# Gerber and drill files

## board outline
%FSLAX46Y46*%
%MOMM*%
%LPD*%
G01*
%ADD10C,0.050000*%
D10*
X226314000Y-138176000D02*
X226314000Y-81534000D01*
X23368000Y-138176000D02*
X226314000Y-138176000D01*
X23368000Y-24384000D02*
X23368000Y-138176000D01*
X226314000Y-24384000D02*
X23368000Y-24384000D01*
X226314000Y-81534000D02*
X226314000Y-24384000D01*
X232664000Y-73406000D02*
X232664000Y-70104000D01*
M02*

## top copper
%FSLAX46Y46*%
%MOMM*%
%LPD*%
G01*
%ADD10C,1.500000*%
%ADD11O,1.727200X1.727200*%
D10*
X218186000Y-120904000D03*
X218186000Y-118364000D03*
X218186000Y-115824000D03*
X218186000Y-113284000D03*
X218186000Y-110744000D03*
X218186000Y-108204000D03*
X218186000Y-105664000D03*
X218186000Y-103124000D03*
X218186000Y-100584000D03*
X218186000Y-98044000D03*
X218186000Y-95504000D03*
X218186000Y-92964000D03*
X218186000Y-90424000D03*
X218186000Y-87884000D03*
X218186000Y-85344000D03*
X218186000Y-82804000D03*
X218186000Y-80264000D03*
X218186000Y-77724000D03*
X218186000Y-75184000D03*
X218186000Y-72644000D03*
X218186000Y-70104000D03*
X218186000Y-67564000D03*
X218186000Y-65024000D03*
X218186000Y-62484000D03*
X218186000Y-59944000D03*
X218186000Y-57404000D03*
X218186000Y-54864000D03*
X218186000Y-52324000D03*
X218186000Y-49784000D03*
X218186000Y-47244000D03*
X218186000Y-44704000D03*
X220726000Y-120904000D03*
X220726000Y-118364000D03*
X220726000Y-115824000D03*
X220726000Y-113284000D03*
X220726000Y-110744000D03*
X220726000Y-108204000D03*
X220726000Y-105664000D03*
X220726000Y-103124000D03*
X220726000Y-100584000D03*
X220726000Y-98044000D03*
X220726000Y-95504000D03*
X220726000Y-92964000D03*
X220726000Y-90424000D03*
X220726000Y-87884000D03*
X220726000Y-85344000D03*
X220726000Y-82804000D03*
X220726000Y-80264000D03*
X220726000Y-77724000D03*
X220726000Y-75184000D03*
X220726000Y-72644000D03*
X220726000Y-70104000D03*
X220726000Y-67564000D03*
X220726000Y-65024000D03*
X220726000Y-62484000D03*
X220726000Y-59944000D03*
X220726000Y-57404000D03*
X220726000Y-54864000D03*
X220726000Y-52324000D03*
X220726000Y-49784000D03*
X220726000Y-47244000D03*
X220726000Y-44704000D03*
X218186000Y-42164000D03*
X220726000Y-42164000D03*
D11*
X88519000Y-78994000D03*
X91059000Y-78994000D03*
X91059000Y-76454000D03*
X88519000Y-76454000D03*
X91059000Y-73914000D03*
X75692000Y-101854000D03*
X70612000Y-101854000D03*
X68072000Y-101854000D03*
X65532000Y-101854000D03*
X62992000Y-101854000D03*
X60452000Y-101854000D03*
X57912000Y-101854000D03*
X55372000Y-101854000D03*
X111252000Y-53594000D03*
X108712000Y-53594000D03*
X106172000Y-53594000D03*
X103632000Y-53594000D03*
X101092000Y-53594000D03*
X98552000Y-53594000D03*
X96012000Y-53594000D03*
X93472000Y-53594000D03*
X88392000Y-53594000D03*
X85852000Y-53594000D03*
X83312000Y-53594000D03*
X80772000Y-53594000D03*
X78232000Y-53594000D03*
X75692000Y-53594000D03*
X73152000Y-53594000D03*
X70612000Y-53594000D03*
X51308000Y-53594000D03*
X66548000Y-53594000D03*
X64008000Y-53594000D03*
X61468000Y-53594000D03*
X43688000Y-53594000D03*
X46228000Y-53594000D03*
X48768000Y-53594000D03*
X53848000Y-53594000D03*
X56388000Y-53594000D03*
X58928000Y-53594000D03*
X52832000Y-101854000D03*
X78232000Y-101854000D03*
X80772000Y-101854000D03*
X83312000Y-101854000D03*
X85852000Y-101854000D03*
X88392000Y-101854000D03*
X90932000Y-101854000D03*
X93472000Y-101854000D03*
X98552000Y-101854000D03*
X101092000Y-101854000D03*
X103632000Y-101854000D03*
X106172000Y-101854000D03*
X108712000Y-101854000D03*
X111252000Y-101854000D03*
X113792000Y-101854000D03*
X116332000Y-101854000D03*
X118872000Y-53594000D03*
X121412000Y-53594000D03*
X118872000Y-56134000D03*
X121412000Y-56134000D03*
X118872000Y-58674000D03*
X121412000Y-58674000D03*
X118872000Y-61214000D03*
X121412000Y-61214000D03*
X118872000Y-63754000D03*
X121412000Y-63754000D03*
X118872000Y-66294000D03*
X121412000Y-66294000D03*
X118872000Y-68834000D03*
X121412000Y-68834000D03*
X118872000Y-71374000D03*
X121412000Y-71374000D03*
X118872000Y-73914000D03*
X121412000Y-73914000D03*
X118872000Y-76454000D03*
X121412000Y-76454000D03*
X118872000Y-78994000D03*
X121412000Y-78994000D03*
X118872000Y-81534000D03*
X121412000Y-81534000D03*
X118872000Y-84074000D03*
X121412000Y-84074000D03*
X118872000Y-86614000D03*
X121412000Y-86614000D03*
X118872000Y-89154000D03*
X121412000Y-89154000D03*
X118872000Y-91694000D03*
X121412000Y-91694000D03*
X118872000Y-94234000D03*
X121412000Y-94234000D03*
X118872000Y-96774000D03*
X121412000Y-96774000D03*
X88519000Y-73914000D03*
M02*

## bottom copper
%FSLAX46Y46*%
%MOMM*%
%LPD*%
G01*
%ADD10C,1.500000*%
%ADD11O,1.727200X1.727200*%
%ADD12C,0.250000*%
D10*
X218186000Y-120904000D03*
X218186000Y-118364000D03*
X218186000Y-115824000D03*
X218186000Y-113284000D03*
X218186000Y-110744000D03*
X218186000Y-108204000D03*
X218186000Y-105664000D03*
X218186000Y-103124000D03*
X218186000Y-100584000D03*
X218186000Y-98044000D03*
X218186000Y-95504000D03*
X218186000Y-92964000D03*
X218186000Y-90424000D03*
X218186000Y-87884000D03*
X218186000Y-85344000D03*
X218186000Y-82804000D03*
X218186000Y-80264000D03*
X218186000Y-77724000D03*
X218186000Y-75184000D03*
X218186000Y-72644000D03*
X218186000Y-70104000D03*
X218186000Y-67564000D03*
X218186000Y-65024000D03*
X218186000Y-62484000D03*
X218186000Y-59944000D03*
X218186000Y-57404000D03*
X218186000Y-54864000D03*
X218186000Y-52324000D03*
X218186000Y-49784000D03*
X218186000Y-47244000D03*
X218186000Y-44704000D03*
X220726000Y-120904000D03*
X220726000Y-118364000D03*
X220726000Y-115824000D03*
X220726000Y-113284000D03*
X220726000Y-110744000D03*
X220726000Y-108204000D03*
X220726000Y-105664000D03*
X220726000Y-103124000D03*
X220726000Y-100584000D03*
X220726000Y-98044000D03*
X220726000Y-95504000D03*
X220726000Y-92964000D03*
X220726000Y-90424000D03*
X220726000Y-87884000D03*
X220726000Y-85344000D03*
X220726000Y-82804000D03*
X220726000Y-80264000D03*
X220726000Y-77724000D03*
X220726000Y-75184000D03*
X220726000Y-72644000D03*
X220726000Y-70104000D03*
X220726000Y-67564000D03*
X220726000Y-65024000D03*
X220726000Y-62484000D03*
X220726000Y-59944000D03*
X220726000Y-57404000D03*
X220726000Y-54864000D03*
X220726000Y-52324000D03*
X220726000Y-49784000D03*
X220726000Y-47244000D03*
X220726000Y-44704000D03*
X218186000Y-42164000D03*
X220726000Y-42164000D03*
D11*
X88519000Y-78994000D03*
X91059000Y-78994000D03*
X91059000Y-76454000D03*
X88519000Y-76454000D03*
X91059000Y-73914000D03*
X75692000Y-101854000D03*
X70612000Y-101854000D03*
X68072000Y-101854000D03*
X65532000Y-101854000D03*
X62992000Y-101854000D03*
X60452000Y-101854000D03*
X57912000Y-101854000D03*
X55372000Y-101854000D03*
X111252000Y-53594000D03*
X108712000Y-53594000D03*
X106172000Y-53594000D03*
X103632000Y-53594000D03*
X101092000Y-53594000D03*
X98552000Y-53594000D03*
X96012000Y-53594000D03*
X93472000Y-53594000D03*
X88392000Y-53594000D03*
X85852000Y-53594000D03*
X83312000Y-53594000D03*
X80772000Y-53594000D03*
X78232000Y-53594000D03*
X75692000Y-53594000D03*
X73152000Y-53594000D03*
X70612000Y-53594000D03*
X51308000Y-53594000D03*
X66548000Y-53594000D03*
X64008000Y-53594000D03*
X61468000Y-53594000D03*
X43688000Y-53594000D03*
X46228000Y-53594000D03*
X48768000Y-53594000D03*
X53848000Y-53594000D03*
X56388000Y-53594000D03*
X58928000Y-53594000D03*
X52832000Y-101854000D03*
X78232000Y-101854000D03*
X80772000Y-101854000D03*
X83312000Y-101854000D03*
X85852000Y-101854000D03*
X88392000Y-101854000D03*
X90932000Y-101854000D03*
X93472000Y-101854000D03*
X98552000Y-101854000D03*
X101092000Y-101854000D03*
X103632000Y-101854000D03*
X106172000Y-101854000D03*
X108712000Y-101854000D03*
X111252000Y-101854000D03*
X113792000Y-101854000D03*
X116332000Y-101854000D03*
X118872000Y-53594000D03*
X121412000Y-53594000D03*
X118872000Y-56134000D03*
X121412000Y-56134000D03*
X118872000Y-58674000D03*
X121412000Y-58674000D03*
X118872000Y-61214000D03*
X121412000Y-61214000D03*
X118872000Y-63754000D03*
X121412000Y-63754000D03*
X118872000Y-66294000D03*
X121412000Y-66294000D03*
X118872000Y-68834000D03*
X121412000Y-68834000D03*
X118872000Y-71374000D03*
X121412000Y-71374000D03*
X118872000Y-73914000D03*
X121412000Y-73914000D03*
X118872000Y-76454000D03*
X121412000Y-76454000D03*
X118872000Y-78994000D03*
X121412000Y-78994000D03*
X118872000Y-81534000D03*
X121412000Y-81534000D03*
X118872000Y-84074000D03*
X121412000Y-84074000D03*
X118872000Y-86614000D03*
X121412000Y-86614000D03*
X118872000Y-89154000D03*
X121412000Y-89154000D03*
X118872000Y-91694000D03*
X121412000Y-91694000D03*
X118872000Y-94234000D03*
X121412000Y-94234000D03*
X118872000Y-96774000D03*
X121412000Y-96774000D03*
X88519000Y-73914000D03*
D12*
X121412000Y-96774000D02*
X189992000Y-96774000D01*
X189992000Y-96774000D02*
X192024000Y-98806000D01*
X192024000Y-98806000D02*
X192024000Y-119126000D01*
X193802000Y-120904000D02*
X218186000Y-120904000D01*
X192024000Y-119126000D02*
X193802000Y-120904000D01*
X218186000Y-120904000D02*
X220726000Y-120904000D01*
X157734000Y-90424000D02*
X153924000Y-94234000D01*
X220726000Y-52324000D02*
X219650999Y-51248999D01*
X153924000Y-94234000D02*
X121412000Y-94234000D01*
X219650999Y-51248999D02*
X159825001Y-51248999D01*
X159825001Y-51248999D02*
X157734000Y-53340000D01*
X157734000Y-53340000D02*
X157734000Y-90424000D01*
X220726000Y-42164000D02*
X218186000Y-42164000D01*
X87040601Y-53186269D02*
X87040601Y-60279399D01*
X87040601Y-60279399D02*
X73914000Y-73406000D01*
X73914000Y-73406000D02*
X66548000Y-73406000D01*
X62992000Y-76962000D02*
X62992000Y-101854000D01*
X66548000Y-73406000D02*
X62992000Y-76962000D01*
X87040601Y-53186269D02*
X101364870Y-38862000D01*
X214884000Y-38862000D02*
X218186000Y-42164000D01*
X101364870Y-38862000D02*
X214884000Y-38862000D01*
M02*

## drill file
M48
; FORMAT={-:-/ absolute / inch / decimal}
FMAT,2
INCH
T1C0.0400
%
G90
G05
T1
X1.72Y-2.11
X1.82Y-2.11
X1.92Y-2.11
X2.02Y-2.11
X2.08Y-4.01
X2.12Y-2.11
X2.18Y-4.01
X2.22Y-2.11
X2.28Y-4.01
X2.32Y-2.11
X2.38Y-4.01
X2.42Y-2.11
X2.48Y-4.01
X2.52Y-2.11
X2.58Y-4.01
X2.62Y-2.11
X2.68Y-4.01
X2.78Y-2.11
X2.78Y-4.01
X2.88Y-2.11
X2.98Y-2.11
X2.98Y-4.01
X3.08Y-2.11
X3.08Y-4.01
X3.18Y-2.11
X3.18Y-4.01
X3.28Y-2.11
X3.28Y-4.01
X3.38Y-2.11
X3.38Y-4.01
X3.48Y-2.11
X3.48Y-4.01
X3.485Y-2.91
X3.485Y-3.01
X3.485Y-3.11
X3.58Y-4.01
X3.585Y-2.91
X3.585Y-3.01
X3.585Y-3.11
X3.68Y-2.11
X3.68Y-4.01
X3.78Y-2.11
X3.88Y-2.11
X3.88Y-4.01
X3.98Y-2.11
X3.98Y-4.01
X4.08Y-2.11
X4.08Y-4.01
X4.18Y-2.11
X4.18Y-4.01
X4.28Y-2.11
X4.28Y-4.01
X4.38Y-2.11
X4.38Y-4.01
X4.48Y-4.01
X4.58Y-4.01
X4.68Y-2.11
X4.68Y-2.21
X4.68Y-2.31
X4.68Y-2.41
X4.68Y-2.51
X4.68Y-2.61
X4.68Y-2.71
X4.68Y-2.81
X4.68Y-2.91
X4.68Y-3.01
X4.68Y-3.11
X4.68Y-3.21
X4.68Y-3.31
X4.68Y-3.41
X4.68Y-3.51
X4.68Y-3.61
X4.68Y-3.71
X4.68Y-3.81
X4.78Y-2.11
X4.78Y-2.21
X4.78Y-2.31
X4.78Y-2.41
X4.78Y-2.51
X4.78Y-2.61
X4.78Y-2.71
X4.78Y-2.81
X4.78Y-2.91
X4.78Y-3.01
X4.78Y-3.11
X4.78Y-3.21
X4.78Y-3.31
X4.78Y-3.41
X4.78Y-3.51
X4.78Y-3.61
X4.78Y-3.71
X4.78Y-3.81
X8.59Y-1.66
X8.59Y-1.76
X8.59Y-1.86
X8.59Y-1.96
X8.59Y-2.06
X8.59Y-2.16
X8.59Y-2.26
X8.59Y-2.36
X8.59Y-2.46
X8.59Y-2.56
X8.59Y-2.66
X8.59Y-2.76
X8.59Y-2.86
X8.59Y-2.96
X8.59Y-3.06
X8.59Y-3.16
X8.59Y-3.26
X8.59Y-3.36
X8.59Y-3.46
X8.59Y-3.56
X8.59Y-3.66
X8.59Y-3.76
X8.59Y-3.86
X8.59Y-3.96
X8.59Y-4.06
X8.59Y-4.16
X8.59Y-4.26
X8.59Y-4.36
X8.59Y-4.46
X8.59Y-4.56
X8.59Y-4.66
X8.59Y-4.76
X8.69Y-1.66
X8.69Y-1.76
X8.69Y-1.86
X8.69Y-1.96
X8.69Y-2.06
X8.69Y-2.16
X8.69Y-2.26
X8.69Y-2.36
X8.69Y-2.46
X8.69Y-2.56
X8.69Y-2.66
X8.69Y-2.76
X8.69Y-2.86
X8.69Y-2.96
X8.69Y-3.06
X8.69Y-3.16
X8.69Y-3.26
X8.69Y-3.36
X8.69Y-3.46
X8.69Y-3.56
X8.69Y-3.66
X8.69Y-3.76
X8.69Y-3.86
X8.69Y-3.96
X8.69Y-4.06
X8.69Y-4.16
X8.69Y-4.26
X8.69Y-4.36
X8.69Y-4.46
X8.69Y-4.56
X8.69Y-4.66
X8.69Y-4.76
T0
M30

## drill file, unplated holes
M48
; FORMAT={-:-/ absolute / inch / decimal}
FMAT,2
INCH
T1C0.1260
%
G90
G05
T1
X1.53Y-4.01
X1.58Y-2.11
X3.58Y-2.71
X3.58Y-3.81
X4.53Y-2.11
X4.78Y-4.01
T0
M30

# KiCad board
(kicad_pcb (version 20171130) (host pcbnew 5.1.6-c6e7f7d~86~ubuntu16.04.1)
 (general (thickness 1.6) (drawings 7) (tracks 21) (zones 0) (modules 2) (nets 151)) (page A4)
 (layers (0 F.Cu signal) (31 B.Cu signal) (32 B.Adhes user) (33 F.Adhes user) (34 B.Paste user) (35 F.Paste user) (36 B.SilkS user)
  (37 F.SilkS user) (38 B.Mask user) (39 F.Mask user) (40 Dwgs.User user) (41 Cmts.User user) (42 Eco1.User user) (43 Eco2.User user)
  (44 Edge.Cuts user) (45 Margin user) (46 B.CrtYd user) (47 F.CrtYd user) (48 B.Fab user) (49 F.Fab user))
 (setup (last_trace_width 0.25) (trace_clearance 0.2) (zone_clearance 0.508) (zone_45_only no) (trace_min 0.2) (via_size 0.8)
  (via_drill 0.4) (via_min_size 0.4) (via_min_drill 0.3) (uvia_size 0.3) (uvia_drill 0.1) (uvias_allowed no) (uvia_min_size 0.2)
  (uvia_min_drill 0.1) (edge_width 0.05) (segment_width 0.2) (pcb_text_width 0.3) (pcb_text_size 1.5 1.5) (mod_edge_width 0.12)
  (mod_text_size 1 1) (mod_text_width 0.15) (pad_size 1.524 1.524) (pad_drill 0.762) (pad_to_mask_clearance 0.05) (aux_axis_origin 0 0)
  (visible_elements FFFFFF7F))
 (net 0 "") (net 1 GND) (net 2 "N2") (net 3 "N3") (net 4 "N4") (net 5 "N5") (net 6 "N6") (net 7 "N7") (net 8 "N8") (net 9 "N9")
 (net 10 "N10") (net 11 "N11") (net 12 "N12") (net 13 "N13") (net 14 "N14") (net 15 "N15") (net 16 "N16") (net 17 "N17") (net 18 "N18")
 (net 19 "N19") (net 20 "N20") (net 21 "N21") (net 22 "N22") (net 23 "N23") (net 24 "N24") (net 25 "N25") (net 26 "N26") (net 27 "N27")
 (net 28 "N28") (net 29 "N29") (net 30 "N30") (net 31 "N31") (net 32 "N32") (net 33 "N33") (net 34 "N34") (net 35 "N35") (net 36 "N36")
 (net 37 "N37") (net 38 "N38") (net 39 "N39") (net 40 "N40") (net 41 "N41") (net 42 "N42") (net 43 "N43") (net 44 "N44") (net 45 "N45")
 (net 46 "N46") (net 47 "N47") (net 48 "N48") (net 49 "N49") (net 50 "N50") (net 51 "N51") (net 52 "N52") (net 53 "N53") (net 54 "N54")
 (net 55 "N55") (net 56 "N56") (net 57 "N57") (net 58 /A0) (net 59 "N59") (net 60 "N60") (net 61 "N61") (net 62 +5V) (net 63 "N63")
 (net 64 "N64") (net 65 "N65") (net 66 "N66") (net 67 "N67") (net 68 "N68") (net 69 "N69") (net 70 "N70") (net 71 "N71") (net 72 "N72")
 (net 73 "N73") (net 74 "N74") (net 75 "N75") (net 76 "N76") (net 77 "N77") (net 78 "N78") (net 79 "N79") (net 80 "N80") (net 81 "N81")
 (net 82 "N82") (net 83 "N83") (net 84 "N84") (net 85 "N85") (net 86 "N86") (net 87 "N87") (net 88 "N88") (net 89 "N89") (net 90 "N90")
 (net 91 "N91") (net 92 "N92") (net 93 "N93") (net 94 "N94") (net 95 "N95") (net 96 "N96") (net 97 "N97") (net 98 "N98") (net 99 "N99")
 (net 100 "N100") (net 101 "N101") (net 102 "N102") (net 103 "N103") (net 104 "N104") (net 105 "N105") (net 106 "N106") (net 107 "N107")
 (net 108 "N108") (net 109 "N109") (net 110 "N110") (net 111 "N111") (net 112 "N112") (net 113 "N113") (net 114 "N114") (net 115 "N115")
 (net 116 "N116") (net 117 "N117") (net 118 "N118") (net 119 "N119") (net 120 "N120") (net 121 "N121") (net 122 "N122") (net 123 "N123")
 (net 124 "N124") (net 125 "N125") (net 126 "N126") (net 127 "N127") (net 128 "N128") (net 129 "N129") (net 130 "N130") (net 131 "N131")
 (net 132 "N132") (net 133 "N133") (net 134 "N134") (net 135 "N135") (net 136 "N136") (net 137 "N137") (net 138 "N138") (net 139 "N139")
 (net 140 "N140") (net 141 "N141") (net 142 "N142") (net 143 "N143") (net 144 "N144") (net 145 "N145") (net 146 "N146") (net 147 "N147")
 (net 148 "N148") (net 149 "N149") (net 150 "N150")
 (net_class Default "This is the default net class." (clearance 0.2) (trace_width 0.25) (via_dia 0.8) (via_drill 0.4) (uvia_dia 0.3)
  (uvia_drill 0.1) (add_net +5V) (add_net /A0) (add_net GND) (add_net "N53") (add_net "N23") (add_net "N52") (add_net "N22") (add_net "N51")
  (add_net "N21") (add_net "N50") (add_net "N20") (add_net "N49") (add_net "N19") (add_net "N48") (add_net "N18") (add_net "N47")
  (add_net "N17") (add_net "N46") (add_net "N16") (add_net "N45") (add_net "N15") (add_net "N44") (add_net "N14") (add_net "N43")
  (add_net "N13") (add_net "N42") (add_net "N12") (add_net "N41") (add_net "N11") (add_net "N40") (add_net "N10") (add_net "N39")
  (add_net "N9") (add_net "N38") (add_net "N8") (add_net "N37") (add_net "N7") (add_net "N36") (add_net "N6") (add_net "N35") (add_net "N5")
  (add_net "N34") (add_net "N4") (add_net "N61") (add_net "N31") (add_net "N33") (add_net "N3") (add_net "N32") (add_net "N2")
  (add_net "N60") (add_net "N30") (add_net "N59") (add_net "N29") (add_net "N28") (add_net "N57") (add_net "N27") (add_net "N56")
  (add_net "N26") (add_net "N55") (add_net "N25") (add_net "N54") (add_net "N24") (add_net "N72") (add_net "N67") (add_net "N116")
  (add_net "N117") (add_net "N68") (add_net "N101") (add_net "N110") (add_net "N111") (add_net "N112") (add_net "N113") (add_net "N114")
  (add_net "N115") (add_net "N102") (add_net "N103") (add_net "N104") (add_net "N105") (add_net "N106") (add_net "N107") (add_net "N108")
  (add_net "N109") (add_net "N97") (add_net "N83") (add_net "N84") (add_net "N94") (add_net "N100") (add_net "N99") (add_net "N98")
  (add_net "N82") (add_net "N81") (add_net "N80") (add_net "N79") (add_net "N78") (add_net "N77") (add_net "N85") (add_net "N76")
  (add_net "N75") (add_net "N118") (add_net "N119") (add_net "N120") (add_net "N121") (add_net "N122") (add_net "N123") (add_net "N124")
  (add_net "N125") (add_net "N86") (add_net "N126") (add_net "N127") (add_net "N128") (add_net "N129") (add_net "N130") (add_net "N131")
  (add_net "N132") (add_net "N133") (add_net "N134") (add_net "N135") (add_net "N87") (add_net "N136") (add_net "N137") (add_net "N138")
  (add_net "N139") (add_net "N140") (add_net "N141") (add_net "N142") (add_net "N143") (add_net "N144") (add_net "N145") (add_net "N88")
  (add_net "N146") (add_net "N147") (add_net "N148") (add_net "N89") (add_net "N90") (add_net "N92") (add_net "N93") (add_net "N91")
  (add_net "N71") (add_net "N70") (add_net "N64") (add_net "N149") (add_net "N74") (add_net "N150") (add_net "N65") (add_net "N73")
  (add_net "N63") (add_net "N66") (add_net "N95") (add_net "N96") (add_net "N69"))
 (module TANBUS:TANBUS (layer F.Cu) (at 219.456 81.534 270)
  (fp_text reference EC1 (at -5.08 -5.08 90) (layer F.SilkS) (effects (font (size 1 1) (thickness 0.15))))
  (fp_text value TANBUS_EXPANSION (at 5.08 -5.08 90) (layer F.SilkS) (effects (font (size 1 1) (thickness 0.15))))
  (pad 32b thru_hole circle (at 39.37 1.27 270) (size 1.5 1.5) (drill 1.016) (layers *.Cu *.Mask F.SilkS) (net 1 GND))
  (pad 31b thru_hole circle (at 36.83 1.27 270) (size 1.5 1.5) (drill 1.016) (layers *.Cu *.Mask F.SilkS) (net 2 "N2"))
  (pad 30b thru_hole circle (at 34.29 1.27 270) (size 1.5 1.5) (drill 1.016) (layers *.Cu *.Mask F.SilkS) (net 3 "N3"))
  (pad 29b thru_hole circle (at 31.75 1.27 270) (size 1.5 1.5) (drill 1.016) (layers *.Cu *.Mask F.SilkS) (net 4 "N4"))
  (pad 28b thru_hole circle (at 29.21 1.27 270) (size 1.5 1.5) (drill 1.016) (layers *.Cu *.Mask F.SilkS) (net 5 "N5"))
  (pad 27b thru_hole circle (at 26.67 1.27 270) (size 1.5 1.5) (drill 1.016) (layers *.Cu *.Mask F.SilkS) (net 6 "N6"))
  (pad 26b thru_hole circle (at 24.13 1.27 270) (size 1.5 1.5) (drill 1.016) (layers *.Cu *.Mask F.SilkS) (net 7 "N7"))
  (pad 25b thru_hole circle (at 21.59 1.27 270) (size 1.5 1.5) (drill 1.016) (layers *.Cu *.Mask F.SilkS) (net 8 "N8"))
  (pad 24b thru_hole circle (at 19.05 1.27 270) (size 1.5 1.5) (drill 1.016) (layers *.Cu *.Mask F.SilkS) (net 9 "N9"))
  (pad 23b thru_hole circle (at 16.51 1.27 270) (size 1.5 1.5) (drill 1.016) (layers *.Cu *.Mask F.SilkS) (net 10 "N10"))
  (pad 22b thru_hole circle (at 13.97 1.27 270) (size 1.5 1.5) (drill 1.016) (layers *.Cu *.Mask F.SilkS) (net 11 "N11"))
  (pad 21b thru_hole circle (at 11.43 1.27 270) (size 1.5 1.5) (drill 1.016) (layers *.Cu *.Mask F.SilkS) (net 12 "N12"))
  (pad 20b thru_hole circle (at 8.89 1.27 270) (size 1.5 1.5) (drill 1.016) (layers *.Cu *.Mask F.SilkS) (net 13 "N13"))
  (pad 19b thru_hole circle (at 6.35 1.27 270) (size 1.5 1.5) (drill 1.016) (layers *.Cu *.Mask F.SilkS) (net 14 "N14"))
  (pad 18b thru_hole circle (at 3.81 1.27 270) (size 1.5 1.5) (drill 1.016) (layers *.Cu *.Mask F.SilkS) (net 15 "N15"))
  (pad 17b thru_hole circle (at 1.27 1.27 270) (size 1.5 1.5) (drill 1.016) (layers *.Cu *.Mask F.SilkS) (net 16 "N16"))
  (pad 16b thru_hole circle (at -1.27 1.27 270) (size 1.5 1.5) (drill 1.016) (layers *.Cu *.Mask F.SilkS) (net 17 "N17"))
  (pad 15b thru_hole circle (at -3.81 1.27 270) (size 1.5 1.5) (drill 1.016) (layers *.Cu *.Mask F.SilkS) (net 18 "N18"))
  (pad 14b thru_hole circle (at -6.35 1.27 270) (size 1.5 1.5) (drill 1.016) (layers *.Cu *.Mask F.SilkS) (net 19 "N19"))
  (pad 13b thru_hole circle (at -8.89 1.27 270) (size 1.5 1.5) (drill 1.016) (layers *.Cu *.Mask F.SilkS) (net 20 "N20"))
  (pad 12b thru_hole circle (at -11.43 1.27 270) (size 1.5 1.5) (drill 1.016) (layers *.Cu *.Mask F.SilkS) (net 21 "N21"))
  (pad 11b thru_hole circle (at -13.97 1.27 270) (size 1.5 1.5) (drill 1.016) (layers *.Cu *.Mask F.SilkS) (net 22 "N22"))
  (pad 10b thru_hole circle (at -16.51 1.27 270) (size 1.5 1.5) (drill 1.016) (layers *.Cu *.Mask F.SilkS) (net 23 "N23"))
  (pad 9b thru_hole circle (at -19.05 1.27 270) (size 1.5 1.5) (drill 1.016) (layers *.Cu *.Mask F.SilkS) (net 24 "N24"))
  (pad 8b thru_hole circle (at -21.59 1.27 270) (size 1.5 1.5) (drill 1.016) (layers *.Cu *.Mask F.SilkS) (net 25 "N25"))
  (pad 7b thru_hole circle (at -24.13 1.27 270) (size 1.5 1.5) (drill 1.016) (layers *.Cu *.Mask F.SilkS) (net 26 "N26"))
  (pad 6b thru_hole circle (at -26.67 1.27 270) (size 1.5 1.5) (drill 1.016) (layers *.Cu *.Mask F.SilkS) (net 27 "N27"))
  (pad 5b thru_hole circle (at -29.21 1.27 270) (size 1.5 1.5) (drill 1.016) (layers *.Cu *.Mask F.SilkS) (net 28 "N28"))
  (pad 4b thru_hole circle (at -31.75 1.27 270) (size 1.5 1.5) (drill 1.016) (layers *.Cu *.Mask F.SilkS) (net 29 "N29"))
  (pad 3b thru_hole circle (at -34.29 1.27 270) (size 1.5 1.5) (drill 1.016) (layers *.Cu *.Mask F.SilkS) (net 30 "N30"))
  (pad 2b thru_hole circle (at -36.83 1.27 270) (size 1.5 1.5) (drill 1.016) (layers *.Cu *.Mask F.SilkS) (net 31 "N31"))
  (pad 32a thru_hole circle (at 39.37 -1.27 270) (size 1.5 1.5) (drill 1.016) (layers *.Cu *.Mask F.SilkS) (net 1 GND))
  (pad 31a thru_hole circle (at 36.83 -1.27 270) (size 1.5 1.5) (drill 1.016) (layers *.Cu *.Mask F.SilkS) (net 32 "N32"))
  (pad 30a thru_hole circle (at 34.29 -1.27 270) (size 1.5 1.5) (drill 1.016) (layers *.Cu *.Mask F.SilkS) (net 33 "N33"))
  (pad 29a thru_hole circle (at 31.75 -1.27 270) (size 1.5 1.5) (drill 1.016) (layers *.Cu *.Mask F.SilkS) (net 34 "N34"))
  (pad 28a thru_hole circle (at 29.21 -1.27 270) (size 1.5 1.5) (drill 1.016) (layers *.Cu *.Mask F.SilkS) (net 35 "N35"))
  (pad 27a thru_hole circle (at 26.67 -1.27 270) (size 1.5 1.5) (drill 1.016) (layers *.Cu *.Mask F.SilkS) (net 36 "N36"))
  (pad 26a thru_hole circle (at 24.13 -1.27 270) (size 1.5 1.5) (drill 1.016) (layers *.Cu *.Mask F.SilkS) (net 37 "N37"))
  (pad 25a thru_hole circle (at 21.59 -1.27 270) (size 1.5 1.5) (drill 1.016) (layers *.Cu *.Mask F.SilkS) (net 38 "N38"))
  (pad 24a thru_hole circle (at 19.05 -1.27 270) (size 1.5 1.5) (drill 1.016) (layers *.Cu *.Mask F.SilkS) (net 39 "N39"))
  (pad 23a thru_hole circle (at 16.51 -1.27 270) (size 1.5 1.5) (drill 1.016) (layers *.Cu *.Mask F.SilkS) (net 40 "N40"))
  (pad 22a thru_hole circle (at 13.97 -1.27 270) (size 1.5 1.5) (drill 1.016) (layers *.Cu *.Mask F.SilkS) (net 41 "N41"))
  (pad 21a thru_hole circle (at 11.43 -1.27 270) (size 1.5 1.5) (drill 1.016) (layers *.Cu *.Mask F.SilkS) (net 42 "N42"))
  (pad 20a thru_hole circle (at 8.89 -1.27 270) (size 1.5 1.5) (drill 1.016) (layers *.Cu *.Mask F.SilkS) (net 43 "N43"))
  (pad 19a thru_hole circle (at 6.35 -1.27 270) (size 1.5 1.5) (drill 1.016) (layers *.Cu *.Mask F.SilkS) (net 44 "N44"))
  (pad 18a thru_hole circle (at 3.81 -1.27 270) (size 1.5 1.5) (drill 1.016) (layers *.Cu *.Mask F.SilkS) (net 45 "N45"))
  (pad 17a thru_hole circle (at 1.27 -1.27 270) (size 1.5 1.5) (drill 1.016) (layers *.Cu *.Mask F.SilkS) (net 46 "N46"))
  (pad 16a thru_hole circle (at -1.27 -1.27 270) (size 1.5 1.5) (drill 1.016) (layers *.Cu *.Mask F.SilkS) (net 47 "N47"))
  (pad 15a thru_hole circle (at -3.81 -1.27 270) (size 1.5 1.5) (drill 1.016) (layers *.Cu *.Mask F.SilkS) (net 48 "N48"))
  (pad 14a thru_hole circle (at -6.35 -1.27 270) (size 1.5 1.5) (drill 1.016) (layers *.Cu *.Mask F.SilkS) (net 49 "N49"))
  (pad 13a thru_hole circle (at -8.89 -1.27 270) (size 1.5 1.5) (drill 1.016) (layers *.Cu *.Mask F.SilkS) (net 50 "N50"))
  (pad 12a thru_hole circle (at -11.43 -1.27 270) (size 1.5 1.5) (drill 1.016) (layers *.Cu *.Mask F.SilkS) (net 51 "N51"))
  (pad 11a thru_hole circle (at -13.97 -1.27 270) (size 1.5 1.5) (drill 1.016) (layers *.Cu *.Mask F.SilkS) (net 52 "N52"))
  (pad 10a thru_hole circle (at -16.51 -1.27 270) (size 1.5 1.5) (drill 1.016) (layers *.Cu *.Mask F.SilkS) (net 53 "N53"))
  (pad 9a thru_hole circle (at -19.05 -1.27 270) (size 1.5 1.5) (drill 1.016) (layers *.Cu *.Mask F.SilkS) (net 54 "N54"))
  (pad 8a thru_hole circle (at -21.59 -1.27 270) (size 1.5 1.5) (drill 1.016) (layers *.Cu *.Mask F.SilkS) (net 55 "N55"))
  (pad 7a thru_hole circle (at -24.13 -1.27 270) (size 1.5 1.5) (drill 1.016) (layers *.Cu *.Mask F.SilkS) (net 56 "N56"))
  (pad 6a thru_hole circle (at -26.67 -1.27 270) (size 1.5 1.5) (drill 1.016) (layers *.Cu *.Mask F.SilkS) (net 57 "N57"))
  (pad 5a thru_hole circle (at -29.21 -1.27 270) (size 1.5 1.5) (drill 1.016) (layers *.Cu *.Mask F.SilkS) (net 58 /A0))
  (pad 4a thru_hole circle (at -31.75 -1.27 270) (size 1.5 1.5) (drill 1.016) (layers *.Cu *.Mask F.SilkS) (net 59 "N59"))
  (pad 3a thru_hole circle (at -34.29 -1.27 270) (size 1.5 1.5) (drill 1.016) (layers *.Cu *.Mask F.SilkS) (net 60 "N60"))
  (pad 2a thru_hole circle (at -36.83 -1.27 270) (size 1.5 1.5) (drill 1.016) (layers *.Cu *.Mask F.SilkS) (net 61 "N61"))
  (pad 1b thru_hole circle (at -39.37 1.27 270) (size 1.5 1.5) (drill 1.016) (layers *.Cu *.Mask F.SilkS) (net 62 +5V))
  (pad 1a thru_hole circle (at -39.37 -1.27 270) (size 1.5 1.5) (drill 1.016) (layers *.Cu *.Mask F.SilkS) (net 62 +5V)))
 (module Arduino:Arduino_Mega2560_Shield (layer F.Cu) (at 24.892 104.394)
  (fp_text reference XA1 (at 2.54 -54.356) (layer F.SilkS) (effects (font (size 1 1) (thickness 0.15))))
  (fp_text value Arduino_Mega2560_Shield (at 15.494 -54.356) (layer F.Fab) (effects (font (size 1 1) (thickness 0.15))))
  (pad RST2 thru_hole oval (at 63.627 -25.4) (size 1.7272 1.7272) (drill 1.016) (layers *.Cu *.Mask) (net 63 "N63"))
  (pad GND4 thru_hole oval (at 66.167 -25.4) (size 1.7272 1.7272) (drill 1.016) (layers *.Cu *.Mask) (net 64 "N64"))
  (pad MOSI thru_hole oval (at 66.167 -27.94) (size 1.7272 1.7272) (drill 1.016) (layers *.Cu *.Mask) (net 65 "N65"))
  (pad SCK thru_hole oval (at 63.627 -27.94) (size 1.7272 1.7272) (drill 1.016) (layers *.Cu *.Mask) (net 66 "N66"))
  (pad 5V2 thru_hole oval (at 66.167 -30.48) (size 1.7272 1.7272) (drill 1.016) (layers *.Cu *.Mask) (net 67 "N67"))
  (pad A0 thru_hole oval (at 50.8 -2.54) (size 1.7272 1.7272) (drill 1.016) (layers *.Cu *.Mask) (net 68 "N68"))
  (pad VIN thru_hole oval (at 45.72 -2.54) (size 1.7272 1.7272) (drill 1.016) (layers *.Cu *.Mask) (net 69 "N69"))
  (pad GND3 thru_hole oval (at 43.18 -2.54) (size 1.7272 1.7272) (drill 1.016) (layers *.Cu *.Mask) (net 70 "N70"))
  (pad GND2 thru_hole oval (at 40.64 -2.54) (size 1.7272 1.7272) (drill 1.016) (layers *.Cu *.Mask) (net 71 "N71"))
  (pad 5V1 thru_hole oval (at 38.1 -2.54) (size 1.7272 1.7272) (drill 1.016) (layers *.Cu *.Mask) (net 62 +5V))
  (pad 3V3 thru_hole oval (at 35.56 -2.54) (size 1.7272 1.7272) (drill 1.016) (layers *.Cu *.Mask) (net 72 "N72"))
  (pad RST1 thru_hole oval (at 33.02 -2.54) (size 1.7272 1.7272) (drill 1.016) (layers *.Cu *.Mask) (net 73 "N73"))
  (pad IORF thru_hole oval (at 30.48 -2.54) (size 1.7272 1.7272) (drill 1.016) (layers *.Cu *.Mask) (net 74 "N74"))
  (pad D21 thru_hole oval (at 86.36 -50.8) (size 1.7272 1.7272) (drill 1.016) (layers *.Cu *.Mask) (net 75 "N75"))
  (pad D20 thru_hole oval (at 83.82 -50.8) (size 1.7272 1.7272) (drill 1.016) (layers *.Cu *.Mask) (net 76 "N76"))
  (pad D19 thru_hole oval (at 81.28 -50.8) (size 1.7272 1.7272) (drill 1.016) (layers *.Cu *.Mask) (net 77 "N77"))
  (pad D18 thru_hole oval (at 78.74 -50.8) (size 1.7272 1.7272) (drill 1.016) (layers *.Cu *.Mask) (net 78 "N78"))
  (pad D17 thru_hole oval (at 76.2 -50.8) (size 1.7272 1.7272) (drill 1.016) (layers *.Cu *.Mask) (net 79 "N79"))
  (pad D16 thru_hole oval (at 73.66 -50.8) (size 1.7272 1.7272) (drill 1.016) (layers *.Cu *.Mask) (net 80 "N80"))
  (pad D15 thru_hole oval (at 71.12 -50.8) (size 1.7272 1.7272) (drill 1.016) (layers *.Cu *.Mask) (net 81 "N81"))
  (pad D14 thru_hole oval (at 68.58 -50.8) (size 1.7272 1.7272) (drill 1.016) (layers *.Cu *.Mask) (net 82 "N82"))
  (pad D0 thru_hole oval (at 63.5 -50.8) (size 1.7272 1.7272) (drill 1.016) (layers *.Cu *.Mask) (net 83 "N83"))
  (pad D1 thru_hole oval (at 60.96 -50.8) (size 1.7272 1.7272) (drill 1.016) (layers *.Cu *.Mask) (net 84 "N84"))
  (pad D2 thru_hole oval (at 58.42 -50.8) (size 1.7272 1.7272) (drill 1.016) (layers *.Cu *.Mask) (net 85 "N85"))
  (pad D3 thru_hole oval (at 55.88 -50.8) (size 1.7272 1.7272) (drill 1.016) (layers *.Cu *.Mask) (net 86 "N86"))
  (pad D4 thru_hole oval (at 53.34 -50.8) (size 1.7272 1.7272) (drill 1.016) (layers *.Cu *.Mask) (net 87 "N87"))
  (pad D5 thru_hole oval (at 50.8 -50.8) (size 1.7272 1.7272) (drill 1.016) (layers *.Cu *.Mask) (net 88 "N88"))
  (pad D6 thru_hole oval (at 48.26 -50.8) (size 1.7272 1.7272) (drill 1.016) (layers *.Cu *.Mask) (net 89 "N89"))
  (pad D7 thru_hole oval (at 45.72 -50.8) (size 1.7272 1.7272) (drill 1.016) (layers *.Cu *.Mask) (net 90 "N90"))
  (pad GND1 thru_hole oval (at 26.416 -50.8) (size 1.7272 1.7272) (drill 1.016) (layers *.Cu *.Mask) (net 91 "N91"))
  (pad D8 thru_hole oval (at 41.656 -50.8) (size 1.7272 1.7272) (drill 1.016) (layers *.Cu *.Mask) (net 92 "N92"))
  (pad D9 thru_hole oval (at 39.116 -50.8) (size 1.7272 1.7272) (drill 1.016) (layers *.Cu *.Mask) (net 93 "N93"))
  (pad D10 thru_hole oval (at 36.576 -50.8) (size 1.7272 1.7272) (drill 1.016) (layers *.Cu *.Mask) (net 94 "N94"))
  (pad "" np_thru_hole circle (at 66.04 -7.62) (size 3.2 3.2) (drill 3.2) (layers *.Cu *.Mask))
  (pad "" np_thru_hole circle (at 66.04 -35.56) (size 3.2 3.2) (drill 3.2) (layers *.Cu *.Mask))
  (pad "" np_thru_hole circle (at 90.17 -50.8) (size 3.2 3.2) (drill 3.2) (layers *.Cu *.Mask))
  (pad "" np_thru_hole circle (at 15.24 -50.8) (size 3.2 3.2) (drill 3.2) (layers *.Cu *.Mask))
  (pad "" np_thru_hole circle (at 96.52 -2.54) (size 3.2 3.2) (drill 3.2) (layers *.Cu *.Mask))
  (pad "" np_thru_hole circle (at 13.97 -2.54) (size 3.2 3.2) (drill 3.2) (layers *.Cu *.Mask))
  (pad SCL thru_hole oval (at 18.796 -50.8) (size 1.7272 1.7272) (drill 1.016) (layers *.Cu *.Mask) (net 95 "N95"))
  (pad SDA thru_hole oval (at 21.336 -50.8) (size 1.7272 1.7272) (drill 1.016) (layers *.Cu *.Mask) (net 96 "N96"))
  (pad AREF thru_hole oval (at 23.876 -50.8) (size 1.7272 1.7272) (drill 1.016) (layers *.Cu *.Mask) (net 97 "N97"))
  (pad D13 thru_hole oval (at 28.956 -50.8) (size 1.7272 1.7272) (drill 1.016) (layers *.Cu *.Mask) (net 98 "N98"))
  (pad D12 thru_hole oval (at 31.496 -50.8) (size 1.7272 1.7272) (drill 1.016) (layers *.Cu *.Mask) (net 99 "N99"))
  (pad D11 thru_hole oval (at 34.036 -50.8) (size 1.7272 1.7272) (drill 1.016) (layers *.Cu *.Mask) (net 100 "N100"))
  (pad "" thru_hole oval (at 27.94 -2.54) (size 1.7272 1.7272) (drill 1.016) (layers *.Cu *.Mask))
  (pad A1 thru_hole oval (at 53.34 -2.54) (size 1.7272 1.7272) (drill 1.016) (layers *.Cu *.Mask) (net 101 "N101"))
  (pad A2 thru_hole oval (at 55.88 -2.54) (size 1.7272 1.7272) (drill 1.016) (layers *.Cu *.Mask) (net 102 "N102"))
  (pad A3 thru_hole oval (at 58.42 -2.54) (size 1.7272 1.7272) (drill 1.016) (layers *.Cu *.Mask) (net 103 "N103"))
  (pad A4 thru_hole oval (at 60.96 -2.54) (size 1.7272 1.7272) (drill 1.016) (layers *.Cu *.Mask) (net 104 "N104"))
  (pad A5 thru_hole oval (at 63.5 -2.54) (size 1.7272 1.7272) (drill 1.016) (layers *.Cu *.Mask) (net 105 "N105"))
  (pad A6 thru_hole oval (at 66.04 -2.54) (size 1.7272 1.7272) (drill 1.016) (layers *.Cu *.Mask) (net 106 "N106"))
  (pad A7 thru_hole oval (at 68.58 -2.54) (size 1.7272 1.7272) (drill 1.016) (layers *.Cu *.Mask) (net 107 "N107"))
  (pad A8 thru_hole oval (at 73.66 -2.54) (size 1.7272 1.7272) (drill 1.016) (layers *.Cu *.Mask) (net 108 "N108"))
  (pad A9 thru_hole oval (at 76.2 -2.54) (size 1.7272 1.7272) (drill 1.016) (layers *.Cu *.Mask) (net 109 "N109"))
  (pad A10 thru_hole oval (at 78.74 -2.54) (size 1.7272 1.7272) (drill 1.016) (layers *.Cu *.Mask) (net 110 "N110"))
  (pad A11 thru_hole oval (at 81.28 -2.54) (size 1.7272 1.7272) (drill 1.016) (layers *.Cu *.Mask) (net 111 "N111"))
  (pad A12 thru_hole oval (at 83.82 -2.54) (size 1.7272 1.7272) (drill 1.016) (layers *.Cu *.Mask) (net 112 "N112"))
  (pad A13 thru_hole oval (at 86.36 -2.54) (size 1.7272 1.7272) (drill 1.016) (layers *.Cu *.Mask) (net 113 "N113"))
  (pad A14 thru_hole oval (at 88.9 -2.54) (size 1.7272 1.7272) (drill 1.016) (layers *.Cu *.Mask) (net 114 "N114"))
  (pad A15 thru_hole oval (at 91.44 -2.54) (size 1.7272 1.7272) (drill 1.016) (layers *.Cu *.Mask) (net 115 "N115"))
  (pad 5V3 thru_hole oval (at 93.98 -50.8) (size 1.7272 1.7272) (drill 1.016) (layers *.Cu *.Mask) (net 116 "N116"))
  (pad 5V4 thru_hole oval (at 96.52 -50.8) (size 1.7272 1.7272) (drill 1.016) (layers *.Cu *.Mask) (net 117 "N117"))
  (pad D22 thru_hole oval (at 93.98 -48.26) (size 1.7272 1.7272) (drill 1.016) (layers *.Cu *.Mask) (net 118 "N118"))
  (pad D23 thru_hole oval (at 96.52 -48.26) (size 1.7272 1.7272) (drill 1.016) (layers *.Cu *.Mask) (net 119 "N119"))
  (pad D24 thru_hole oval (at 93.98 -45.72) (size 1.7272 1.7272) (drill 1.016) (layers *.Cu *.Mask) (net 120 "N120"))
  (pad D25 thru_hole oval (at 96.52 -45.72) (size 1.7272 1.7272) (drill 1.016) (layers *.Cu *.Mask) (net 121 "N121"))
  (pad D26 thru_hole oval (at 93.98 -43.18) (size 1.7272 1.7272) (drill 1.016) (layers *.Cu *.Mask) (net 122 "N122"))
  (pad D27 thru_hole oval (at 96.52 -43.18) (size 1.7272 1.7272) (drill 1.016) (layers *.Cu *.Mask) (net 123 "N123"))
  (pad D28 thru_hole oval (at 93.98 -40.64) (size 1.7272 1.7272) (drill 1.016) (layers *.Cu *.Mask) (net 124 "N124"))
  (pad D29 thru_hole oval (at 96.52 -40.64) (size 1.7272 1.7272) (drill 1.016) (layers *.Cu *.Mask) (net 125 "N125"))
  (pad D30 thru_hole oval (at 93.98 -38.1) (size 1.7272 1.7272) (drill 1.016) (layers *.Cu *.Mask) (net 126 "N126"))
  (pad D31 thru_hole oval (at 96.52 -38.1) (size 1.7272 1.7272) (drill 1.016) (layers *.Cu *.Mask) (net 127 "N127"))
  (pad D32 thru_hole oval (at 93.98 -35.56) (size 1.7272 1.7272) (drill 1.016) (layers *.Cu *.Mask) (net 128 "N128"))
  (pad D33 thru_hole oval (at 96.52 -35.56) (size 1.7272 1.7272) (drill 1.016) (layers *.Cu *.Mask) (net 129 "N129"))
  (pad D34 thru_hole oval (at 93.98 -33.02) (size 1.7272 1.7272) (drill 1.016) (layers *.Cu *.Mask) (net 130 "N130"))
  (pad D35 thru_hole oval (at 96.52 -33.02) (size 1.7272 1.7272) (drill 1.016) (layers *.Cu *.Mask) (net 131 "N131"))
  (pad D36 thru_hole oval (at 93.98 -30.48) (size 1.7272 1.7272) (drill 1.016) (layers *.Cu *.Mask) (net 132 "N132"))
  (pad D37 thru_hole oval (at 96.52 -30.48) (size 1.7272 1.7272) (drill 1.016) (layers *.Cu *.Mask) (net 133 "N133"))
  (pad D38 thru_hole oval (at 93.98 -27.94) (size 1.7272 1.7272) (drill 1.016) (layers *.Cu *.Mask) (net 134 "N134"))
  (pad D39 thru_hole oval (at 96.52 -27.94) (size 1.7272 1.7272) (drill 1.016) (layers *.Cu *.Mask) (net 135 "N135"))
  (pad D40 thru_hole oval (at 93.98 -25.4) (size 1.7272 1.7272) (drill 1.016) (layers *.Cu *.Mask) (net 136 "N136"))
  (pad D41 thru_hole oval (at 96.52 -25.4) (size 1.7272 1.7272) (drill 1.016) (layers *.Cu *.Mask) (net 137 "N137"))
  (pad D42 thru_hole oval (at 93.98 -22.86) (size 1.7272 1.7272) (drill 1.016) (layers *.Cu *.Mask) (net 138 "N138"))
  (pad D43 thru_hole oval (at 96.52 -22.86) (size 1.7272 1.7272) (drill 1.016) (layers *.Cu *.Mask) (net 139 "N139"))
  (pad D44 thru_hole oval (at 93.98 -20.32) (size 1.7272 1.7272) (drill 1.016) (layers *.Cu *.Mask) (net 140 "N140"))
  (pad D45 thru_hole oval (at 96.52 -20.32) (size 1.7272 1.7272) (drill 1.016) (layers *.Cu *.Mask) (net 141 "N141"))
  (pad D46 thru_hole oval (at 93.98 -17.78) (size 1.7272 1.7272) (drill 1.016) (layers *.Cu *.Mask) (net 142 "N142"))
  (pad D47 thru_hole oval (at 96.52 -17.78) (size 1.7272 1.7272) (drill 1.016) (layers *.Cu *.Mask) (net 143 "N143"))
  (pad D48 thru_hole oval (at 93.98 -15.24) (size 1.7272 1.7272) (drill 1.016) (layers *.Cu *.Mask) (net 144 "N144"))
  (pad D49 thru_hole oval (at 96.52 -15.24) (size 1.7272 1.7272) (drill 1.016) (layers *.Cu *.Mask) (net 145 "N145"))
  (pad D50 thru_hole oval (at 93.98 -12.7) (size 1.7272 1.7272) (drill 1.016) (layers *.Cu *.Mask) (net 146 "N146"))
  (pad D51 thru_hole oval (at 96.52 -12.7) (size 1.7272 1.7272) (drill 1.016) (layers *.Cu *.Mask) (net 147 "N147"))
  (pad D52 thru_hole oval (at 93.98 -10.16) (size 1.7272 1.7272) (drill 1.016) (layers *.Cu *.Mask) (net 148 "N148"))
  (pad D53 thru_hole oval (at 96.52 -10.16) (size 1.7272 1.7272) (drill 1.016) (layers *.Cu *.Mask) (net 58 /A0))
  (pad GND5 thru_hole oval (at 93.98 -7.62) (size 1.7272 1.7272) (drill 1.016) (layers *.Cu *.Mask) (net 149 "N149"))
  (pad GND6 thru_hole oval (at 96.52 -7.62) (size 1.7272 1.7272) (drill 1.016) (layers *.Cu *.Mask) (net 1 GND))
  (pad MISO thru_hole oval (at 63.627 -30.48) (size 1.7272 1.7272) (drill 1.016) (layers *.Cu *.Mask) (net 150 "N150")))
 (gr_line (start 226.314 138.176) (end 226.314 81.534) (layer Edge.Cuts) (width 0.05))
 (gr_line (start 23.368 138.176) (end 226.314 138.176) (layer Edge.Cuts) (width 0.05))
 (gr_line (start 23.368 24.384) (end 23.368 138.176) (layer Edge.Cuts) (width 0.05))
 (gr_line (start 226.314 24.384) (end 23.368 24.384) (layer Edge.Cuts) (width 0.05))
 (gr_line (start 226.314 81.534) (end 226.314 24.384) (layer Edge.Cuts) (width 0.05))
 (gr_line (start 232.664 73.406) (end 232.664 70.104) (layer Edge.Cuts) (width 0.05))
 (segment (start 121.412 96.774) (end 189.992 96.774) (width 0.25) (layer B.Cu) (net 1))
 (segment (start 189.992 96.774) (end 192.024 98.806) (width 0.25) (layer B.Cu) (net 1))
 (segment (start 192.024 98.806) (end 192.024 119.126) (width 0.25) (layer B.Cu) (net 1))
 (segment (start 193.802 120.904) (end 218.186 120.904) (width 0.25) (layer B.Cu) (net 1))
 (segment (start 192.024 119.126) (end 193.802 120.904) (width 0.25) (layer B.Cu) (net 1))
 (segment (start 218.186 120.904) (end 220.726 120.904) (width 0.25) (layer B.Cu) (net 1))
 (segment (start 157.734 90.424) (end 153.924 94.234) (width 0.25) (layer B.Cu) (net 58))
 (segment (start 220.726 52.324) (end 219.650999 51.248999) (width 0.25) (layer B.Cu) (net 58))
 (segment (start 153.924 94.234) (end 121.412 94.234) (width 0.25) (layer B.Cu) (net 58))
 (segment (start 219.650999 51.248999) (end 159.825001 51.248999) (width 0.25) (layer B.Cu) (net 58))
 (segment (start 159.825001 51.248999) (end 157.734 53.34) (width 0.25) (layer B.Cu) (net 58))
 (segment (start 157.734 53.34) (end 157.734 90.424) (width 0.25) (layer B.Cu) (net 58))
 (segment (start 220.726 42.164) (end 218.186 42.164) (width 0.25) (layer B.Cu) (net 62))
 (segment (start 87.040601 53.186269) (end 87.040601 60.279399) (width 0.25) (layer B.Cu) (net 62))
 (segment (start 87.040601 60.279399) (end 73.914 73.406) (width 0.25) (layer B.Cu) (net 62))
 (segment (start 73.914 73.406) (end 66.548 73.406) (width 0.25) (layer B.Cu) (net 62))
 (segment (start 62.992 76.962) (end 62.992 101.854) (width 0.25) (layer B.Cu) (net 62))
 (segment (start 66.548 73.406) (end 62.992 76.962) (width 0.25) (layer B.Cu) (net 62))
 (segment (start 87.040601 53.186269) (end 101.36487 38.862) (width 0.25) (layer B.Cu) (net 62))
 (segment (start 214.884 38.862) (end 218.186 42.164) (width 0.25) (layer B.Cu) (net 62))
 (segment (start 101.36487 38.862) (end 214.884 38.862) (width 0.25) (layer B.Cu) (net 62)))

